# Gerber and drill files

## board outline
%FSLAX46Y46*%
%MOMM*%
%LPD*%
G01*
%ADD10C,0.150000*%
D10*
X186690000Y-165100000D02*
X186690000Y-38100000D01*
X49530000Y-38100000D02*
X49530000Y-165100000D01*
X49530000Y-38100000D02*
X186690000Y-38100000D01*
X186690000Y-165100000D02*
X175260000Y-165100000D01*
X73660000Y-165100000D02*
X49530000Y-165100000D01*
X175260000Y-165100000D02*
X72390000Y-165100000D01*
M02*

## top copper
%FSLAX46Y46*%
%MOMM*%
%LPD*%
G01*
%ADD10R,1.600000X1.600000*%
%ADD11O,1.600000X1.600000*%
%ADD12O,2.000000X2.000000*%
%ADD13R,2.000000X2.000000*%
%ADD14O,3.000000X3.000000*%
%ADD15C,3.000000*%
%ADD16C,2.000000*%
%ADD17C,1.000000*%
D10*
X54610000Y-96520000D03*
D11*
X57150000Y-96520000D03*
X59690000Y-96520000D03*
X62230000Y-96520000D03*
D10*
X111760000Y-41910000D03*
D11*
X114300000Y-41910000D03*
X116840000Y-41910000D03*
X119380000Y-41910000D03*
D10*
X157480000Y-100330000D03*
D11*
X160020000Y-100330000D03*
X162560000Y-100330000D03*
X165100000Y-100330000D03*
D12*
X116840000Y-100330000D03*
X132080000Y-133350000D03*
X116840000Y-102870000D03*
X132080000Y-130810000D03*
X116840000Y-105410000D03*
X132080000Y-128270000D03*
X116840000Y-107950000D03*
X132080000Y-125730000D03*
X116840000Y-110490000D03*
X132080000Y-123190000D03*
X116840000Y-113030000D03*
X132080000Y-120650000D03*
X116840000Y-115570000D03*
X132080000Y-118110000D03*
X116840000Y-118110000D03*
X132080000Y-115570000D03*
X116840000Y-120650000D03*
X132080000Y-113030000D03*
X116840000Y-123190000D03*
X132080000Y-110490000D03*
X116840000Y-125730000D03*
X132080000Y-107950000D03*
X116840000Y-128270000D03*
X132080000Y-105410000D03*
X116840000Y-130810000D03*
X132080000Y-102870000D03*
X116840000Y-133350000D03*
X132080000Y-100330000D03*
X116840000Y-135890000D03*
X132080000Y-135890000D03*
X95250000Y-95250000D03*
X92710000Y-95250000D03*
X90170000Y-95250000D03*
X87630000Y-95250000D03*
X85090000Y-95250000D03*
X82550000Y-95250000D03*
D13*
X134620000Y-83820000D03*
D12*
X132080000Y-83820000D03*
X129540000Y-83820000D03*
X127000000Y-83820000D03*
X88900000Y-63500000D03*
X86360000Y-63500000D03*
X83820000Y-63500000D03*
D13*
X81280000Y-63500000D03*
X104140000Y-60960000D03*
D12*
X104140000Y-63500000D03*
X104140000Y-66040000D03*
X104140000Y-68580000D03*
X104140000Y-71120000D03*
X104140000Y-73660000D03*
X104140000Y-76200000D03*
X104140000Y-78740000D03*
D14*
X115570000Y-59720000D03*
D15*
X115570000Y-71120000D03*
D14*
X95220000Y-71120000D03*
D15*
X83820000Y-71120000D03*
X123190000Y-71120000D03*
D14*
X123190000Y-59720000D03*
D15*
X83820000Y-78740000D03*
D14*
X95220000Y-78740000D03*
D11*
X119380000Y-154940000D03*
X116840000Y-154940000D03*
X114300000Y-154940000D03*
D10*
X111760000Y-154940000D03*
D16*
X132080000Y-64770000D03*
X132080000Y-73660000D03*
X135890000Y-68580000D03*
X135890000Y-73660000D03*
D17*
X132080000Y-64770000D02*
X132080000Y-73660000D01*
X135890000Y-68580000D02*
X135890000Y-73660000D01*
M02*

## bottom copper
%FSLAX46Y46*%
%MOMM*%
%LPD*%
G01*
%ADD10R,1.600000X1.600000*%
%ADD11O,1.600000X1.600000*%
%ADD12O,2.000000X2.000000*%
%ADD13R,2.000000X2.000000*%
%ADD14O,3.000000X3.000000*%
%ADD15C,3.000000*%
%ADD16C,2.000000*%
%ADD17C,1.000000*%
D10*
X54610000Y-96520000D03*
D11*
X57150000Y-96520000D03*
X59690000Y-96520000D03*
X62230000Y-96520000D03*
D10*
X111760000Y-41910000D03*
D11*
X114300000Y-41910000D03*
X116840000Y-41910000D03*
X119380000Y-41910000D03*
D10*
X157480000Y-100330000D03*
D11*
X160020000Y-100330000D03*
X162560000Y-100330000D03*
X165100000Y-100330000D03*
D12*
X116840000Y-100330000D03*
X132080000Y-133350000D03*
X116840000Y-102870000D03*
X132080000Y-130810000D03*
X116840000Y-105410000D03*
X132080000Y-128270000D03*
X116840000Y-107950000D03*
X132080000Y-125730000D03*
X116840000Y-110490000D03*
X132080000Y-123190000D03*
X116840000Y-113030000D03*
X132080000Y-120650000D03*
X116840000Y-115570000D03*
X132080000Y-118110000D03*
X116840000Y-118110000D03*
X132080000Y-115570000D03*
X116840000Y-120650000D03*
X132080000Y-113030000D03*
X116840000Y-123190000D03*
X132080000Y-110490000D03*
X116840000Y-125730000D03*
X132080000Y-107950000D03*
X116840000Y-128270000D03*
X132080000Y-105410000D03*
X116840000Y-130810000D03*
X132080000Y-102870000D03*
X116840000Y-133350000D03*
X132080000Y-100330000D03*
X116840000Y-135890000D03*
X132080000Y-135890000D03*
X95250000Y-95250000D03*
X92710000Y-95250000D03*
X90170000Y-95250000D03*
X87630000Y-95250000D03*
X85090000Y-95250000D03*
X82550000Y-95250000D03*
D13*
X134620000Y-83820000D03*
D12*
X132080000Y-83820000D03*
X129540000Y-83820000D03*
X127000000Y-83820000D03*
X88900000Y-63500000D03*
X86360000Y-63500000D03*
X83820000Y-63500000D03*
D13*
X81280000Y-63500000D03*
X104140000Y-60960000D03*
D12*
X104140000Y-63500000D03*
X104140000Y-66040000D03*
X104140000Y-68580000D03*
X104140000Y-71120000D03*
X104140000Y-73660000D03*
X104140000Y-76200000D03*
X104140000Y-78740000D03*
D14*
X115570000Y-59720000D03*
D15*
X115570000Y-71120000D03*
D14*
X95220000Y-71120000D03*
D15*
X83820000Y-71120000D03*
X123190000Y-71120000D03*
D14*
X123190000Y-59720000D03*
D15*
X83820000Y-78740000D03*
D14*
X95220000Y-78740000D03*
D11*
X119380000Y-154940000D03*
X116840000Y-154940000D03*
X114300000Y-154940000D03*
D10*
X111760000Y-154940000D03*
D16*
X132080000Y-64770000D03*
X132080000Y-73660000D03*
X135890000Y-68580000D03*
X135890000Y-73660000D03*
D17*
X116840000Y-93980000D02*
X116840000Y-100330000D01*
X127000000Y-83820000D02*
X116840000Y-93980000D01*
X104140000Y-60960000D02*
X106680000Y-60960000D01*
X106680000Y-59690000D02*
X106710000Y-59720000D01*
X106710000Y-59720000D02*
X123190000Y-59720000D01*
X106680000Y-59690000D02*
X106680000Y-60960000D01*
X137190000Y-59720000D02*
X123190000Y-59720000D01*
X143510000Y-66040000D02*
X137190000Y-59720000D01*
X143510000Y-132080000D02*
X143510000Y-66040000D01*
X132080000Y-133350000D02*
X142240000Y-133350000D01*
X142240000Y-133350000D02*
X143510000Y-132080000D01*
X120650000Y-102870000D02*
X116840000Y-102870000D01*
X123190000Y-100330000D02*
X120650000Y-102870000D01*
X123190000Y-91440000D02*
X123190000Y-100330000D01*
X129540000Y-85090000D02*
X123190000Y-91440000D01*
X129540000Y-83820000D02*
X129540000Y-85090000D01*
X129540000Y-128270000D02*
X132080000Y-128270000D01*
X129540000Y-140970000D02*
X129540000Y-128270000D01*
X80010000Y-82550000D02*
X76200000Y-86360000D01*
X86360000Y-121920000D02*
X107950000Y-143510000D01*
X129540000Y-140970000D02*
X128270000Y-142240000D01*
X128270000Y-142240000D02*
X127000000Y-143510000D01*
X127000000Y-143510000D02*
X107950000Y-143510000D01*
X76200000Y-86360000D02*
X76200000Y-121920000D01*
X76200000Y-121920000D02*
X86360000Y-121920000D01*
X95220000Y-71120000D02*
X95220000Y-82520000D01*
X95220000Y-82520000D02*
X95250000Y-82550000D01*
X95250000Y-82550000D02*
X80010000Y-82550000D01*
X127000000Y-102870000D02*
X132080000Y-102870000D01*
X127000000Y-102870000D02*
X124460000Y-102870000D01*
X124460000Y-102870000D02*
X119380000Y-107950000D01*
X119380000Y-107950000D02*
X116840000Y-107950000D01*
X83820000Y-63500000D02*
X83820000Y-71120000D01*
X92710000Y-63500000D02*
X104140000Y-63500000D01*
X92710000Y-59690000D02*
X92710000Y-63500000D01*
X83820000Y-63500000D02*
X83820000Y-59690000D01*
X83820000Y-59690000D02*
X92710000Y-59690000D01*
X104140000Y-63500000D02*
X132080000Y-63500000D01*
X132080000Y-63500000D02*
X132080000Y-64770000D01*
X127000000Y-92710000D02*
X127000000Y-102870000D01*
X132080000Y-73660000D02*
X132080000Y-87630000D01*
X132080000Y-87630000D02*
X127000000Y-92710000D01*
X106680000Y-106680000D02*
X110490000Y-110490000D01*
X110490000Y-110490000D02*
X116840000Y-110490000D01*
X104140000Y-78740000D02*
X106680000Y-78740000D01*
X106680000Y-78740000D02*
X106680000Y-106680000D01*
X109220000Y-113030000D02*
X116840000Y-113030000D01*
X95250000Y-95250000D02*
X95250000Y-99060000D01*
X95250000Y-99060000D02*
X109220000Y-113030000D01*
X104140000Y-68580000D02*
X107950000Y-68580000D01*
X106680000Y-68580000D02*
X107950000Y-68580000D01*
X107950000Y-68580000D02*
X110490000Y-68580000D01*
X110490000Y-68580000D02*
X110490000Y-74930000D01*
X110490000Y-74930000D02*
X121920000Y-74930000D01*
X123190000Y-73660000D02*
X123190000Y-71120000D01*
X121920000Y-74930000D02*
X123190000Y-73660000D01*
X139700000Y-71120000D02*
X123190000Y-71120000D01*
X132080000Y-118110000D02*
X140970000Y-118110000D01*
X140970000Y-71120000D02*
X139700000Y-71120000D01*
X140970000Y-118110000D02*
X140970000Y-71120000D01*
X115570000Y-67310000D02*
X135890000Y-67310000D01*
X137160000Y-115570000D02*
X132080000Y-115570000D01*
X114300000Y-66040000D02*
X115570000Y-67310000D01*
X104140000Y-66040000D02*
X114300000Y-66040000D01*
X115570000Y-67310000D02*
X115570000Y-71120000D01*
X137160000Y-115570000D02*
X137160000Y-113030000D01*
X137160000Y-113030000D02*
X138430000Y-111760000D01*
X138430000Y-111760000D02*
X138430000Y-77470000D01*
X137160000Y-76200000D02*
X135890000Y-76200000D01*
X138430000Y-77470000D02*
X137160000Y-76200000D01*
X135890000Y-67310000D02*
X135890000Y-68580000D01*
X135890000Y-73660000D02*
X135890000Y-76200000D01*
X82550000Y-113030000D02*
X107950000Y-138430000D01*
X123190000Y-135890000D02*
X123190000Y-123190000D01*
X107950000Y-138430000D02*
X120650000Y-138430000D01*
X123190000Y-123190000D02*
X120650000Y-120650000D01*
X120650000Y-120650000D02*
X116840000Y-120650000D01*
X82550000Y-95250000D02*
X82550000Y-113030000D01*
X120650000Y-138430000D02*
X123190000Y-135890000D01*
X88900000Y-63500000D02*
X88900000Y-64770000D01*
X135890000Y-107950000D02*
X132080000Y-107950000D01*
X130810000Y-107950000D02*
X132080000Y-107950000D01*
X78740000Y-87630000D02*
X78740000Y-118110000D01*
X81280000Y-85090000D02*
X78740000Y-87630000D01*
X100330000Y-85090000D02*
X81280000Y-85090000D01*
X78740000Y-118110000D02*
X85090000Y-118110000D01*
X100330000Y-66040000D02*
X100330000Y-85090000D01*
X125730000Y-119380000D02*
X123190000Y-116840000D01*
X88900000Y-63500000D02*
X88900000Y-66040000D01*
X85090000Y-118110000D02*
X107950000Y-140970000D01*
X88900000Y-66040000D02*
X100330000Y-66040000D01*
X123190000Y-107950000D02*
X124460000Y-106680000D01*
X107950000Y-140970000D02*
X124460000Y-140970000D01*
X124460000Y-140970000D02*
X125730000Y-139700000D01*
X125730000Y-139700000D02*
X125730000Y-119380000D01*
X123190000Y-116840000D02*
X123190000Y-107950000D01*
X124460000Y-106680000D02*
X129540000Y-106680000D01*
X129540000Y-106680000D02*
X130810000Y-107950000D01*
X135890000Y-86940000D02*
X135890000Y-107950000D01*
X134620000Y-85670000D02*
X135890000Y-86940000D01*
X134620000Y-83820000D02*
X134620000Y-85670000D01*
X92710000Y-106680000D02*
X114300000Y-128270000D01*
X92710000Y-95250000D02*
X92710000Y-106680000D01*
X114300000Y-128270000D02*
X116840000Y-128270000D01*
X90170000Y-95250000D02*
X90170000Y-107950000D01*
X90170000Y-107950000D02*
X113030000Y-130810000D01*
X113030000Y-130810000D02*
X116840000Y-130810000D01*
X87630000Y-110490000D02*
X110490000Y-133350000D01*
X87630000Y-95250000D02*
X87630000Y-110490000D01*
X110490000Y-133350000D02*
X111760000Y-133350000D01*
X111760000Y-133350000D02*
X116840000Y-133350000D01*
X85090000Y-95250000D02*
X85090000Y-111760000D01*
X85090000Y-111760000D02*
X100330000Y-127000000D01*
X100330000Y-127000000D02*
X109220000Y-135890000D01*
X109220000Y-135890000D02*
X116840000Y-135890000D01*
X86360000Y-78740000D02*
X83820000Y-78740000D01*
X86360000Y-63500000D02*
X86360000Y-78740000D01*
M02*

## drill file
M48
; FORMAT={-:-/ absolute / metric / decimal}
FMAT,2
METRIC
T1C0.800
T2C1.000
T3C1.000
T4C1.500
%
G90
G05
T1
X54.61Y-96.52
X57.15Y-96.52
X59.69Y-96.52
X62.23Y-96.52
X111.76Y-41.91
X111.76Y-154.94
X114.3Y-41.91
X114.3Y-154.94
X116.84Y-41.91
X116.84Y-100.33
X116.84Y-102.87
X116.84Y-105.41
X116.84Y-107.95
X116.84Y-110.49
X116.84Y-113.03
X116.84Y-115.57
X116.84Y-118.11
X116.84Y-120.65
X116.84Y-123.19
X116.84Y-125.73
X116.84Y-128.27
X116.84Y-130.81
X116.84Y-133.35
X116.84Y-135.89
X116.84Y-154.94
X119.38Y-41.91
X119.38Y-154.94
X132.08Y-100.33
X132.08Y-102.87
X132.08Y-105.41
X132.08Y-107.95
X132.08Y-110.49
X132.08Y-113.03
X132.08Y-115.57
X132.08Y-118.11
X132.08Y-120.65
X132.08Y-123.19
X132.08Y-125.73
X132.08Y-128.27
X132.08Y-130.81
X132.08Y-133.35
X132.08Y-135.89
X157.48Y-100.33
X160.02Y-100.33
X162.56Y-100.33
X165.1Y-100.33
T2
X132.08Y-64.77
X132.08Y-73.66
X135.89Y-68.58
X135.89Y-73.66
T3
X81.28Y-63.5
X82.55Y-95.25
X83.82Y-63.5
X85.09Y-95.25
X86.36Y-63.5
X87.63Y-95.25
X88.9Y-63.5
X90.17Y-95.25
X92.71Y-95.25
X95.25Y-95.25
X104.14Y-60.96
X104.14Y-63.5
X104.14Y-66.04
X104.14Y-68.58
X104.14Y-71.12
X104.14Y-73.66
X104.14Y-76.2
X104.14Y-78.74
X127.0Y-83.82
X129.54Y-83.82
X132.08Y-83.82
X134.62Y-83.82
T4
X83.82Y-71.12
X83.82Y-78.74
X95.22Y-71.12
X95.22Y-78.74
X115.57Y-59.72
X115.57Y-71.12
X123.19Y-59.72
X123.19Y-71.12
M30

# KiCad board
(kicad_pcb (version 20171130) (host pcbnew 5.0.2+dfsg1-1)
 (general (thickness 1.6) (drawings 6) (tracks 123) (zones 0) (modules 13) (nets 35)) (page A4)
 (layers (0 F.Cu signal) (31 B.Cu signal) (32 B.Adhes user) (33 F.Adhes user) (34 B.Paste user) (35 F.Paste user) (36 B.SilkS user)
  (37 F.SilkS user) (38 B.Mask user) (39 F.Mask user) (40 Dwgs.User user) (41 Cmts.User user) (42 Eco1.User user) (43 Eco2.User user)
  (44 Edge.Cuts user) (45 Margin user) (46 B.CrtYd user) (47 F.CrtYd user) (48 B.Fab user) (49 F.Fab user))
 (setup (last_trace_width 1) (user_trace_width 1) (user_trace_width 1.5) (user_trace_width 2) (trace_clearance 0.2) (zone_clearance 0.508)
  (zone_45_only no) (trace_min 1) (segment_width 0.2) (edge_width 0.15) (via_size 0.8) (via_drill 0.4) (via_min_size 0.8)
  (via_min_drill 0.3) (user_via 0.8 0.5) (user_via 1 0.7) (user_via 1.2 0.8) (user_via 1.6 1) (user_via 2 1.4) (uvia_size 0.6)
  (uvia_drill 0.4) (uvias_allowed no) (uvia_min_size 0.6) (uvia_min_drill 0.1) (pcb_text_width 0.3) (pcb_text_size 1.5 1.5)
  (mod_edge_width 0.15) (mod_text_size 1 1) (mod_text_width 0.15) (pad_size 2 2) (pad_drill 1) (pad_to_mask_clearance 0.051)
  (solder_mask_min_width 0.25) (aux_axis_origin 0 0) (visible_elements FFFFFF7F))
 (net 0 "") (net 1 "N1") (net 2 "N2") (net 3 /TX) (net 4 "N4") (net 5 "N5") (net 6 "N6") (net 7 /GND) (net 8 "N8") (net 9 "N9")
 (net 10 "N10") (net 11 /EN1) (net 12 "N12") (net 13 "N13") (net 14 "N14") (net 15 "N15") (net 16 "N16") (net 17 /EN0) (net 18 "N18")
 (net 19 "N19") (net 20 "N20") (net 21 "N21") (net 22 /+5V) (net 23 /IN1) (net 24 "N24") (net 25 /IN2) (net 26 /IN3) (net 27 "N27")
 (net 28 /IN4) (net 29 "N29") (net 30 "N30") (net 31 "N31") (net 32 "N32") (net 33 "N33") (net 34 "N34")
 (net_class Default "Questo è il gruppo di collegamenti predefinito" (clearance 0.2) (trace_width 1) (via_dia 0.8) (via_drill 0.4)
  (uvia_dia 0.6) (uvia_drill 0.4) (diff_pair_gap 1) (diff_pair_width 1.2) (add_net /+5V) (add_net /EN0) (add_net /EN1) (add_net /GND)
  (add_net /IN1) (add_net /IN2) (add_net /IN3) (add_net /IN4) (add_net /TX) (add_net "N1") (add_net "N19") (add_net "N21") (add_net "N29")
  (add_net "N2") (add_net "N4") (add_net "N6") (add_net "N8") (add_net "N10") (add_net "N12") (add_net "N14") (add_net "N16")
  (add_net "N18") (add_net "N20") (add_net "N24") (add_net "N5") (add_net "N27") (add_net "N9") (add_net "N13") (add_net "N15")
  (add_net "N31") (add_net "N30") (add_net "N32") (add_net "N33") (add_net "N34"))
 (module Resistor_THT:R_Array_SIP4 (layer F.Cu) (at 54.61 96.52)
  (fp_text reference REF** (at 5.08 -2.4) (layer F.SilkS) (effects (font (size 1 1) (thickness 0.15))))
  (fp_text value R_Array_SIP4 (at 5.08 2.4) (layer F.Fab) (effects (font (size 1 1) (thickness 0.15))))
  (pad 1 thru_hole rect (at 0 0) (size 1.6 1.6) (drill 0.8) (layers *.Cu *.Mask))
  (pad 2 thru_hole oval (at 2.54 0) (size 1.6 1.6) (drill 0.8) (layers *.Cu *.Mask))
  (pad 3 thru_hole oval (at 5.08 0) (size 1.6 1.6) (drill 0.8) (layers *.Cu *.Mask))
  (pad 4 thru_hole oval (at 7.62 0) (size 1.6 1.6) (drill 0.8) (layers *.Cu *.Mask)))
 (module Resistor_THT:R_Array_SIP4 (layer F.Cu) (at 111.76 41.91)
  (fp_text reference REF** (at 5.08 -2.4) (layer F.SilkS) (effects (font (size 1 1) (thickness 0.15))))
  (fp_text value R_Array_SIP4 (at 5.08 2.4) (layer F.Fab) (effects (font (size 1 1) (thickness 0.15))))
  (pad 1 thru_hole rect (at 0 0) (size 1.6 1.6) (drill 0.8) (layers *.Cu *.Mask))
  (pad 2 thru_hole oval (at 2.54 0) (size 1.6 1.6) (drill 0.8) (layers *.Cu *.Mask))
  (pad 3 thru_hole oval (at 5.08 0) (size 1.6 1.6) (drill 0.8) (layers *.Cu *.Mask))
  (pad 4 thru_hole oval (at 7.62 0) (size 1.6 1.6) (drill 0.8) (layers *.Cu *.Mask)))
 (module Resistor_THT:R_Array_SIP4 (layer F.Cu) (at 157.48 100.33)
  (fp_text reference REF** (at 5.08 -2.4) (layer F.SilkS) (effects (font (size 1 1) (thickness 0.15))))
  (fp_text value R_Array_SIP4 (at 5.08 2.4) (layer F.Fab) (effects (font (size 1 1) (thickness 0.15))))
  (pad 1 thru_hole rect (at 0 0) (size 1.6 1.6) (drill 0.8) (layers *.Cu *.Mask))
  (pad 2 thru_hole oval (at 2.54 0) (size 1.6 1.6) (drill 0.8) (layers *.Cu *.Mask))
  (pad 3 thru_hole oval (at 5.08 0) (size 1.6 1.6) (drill 0.8) (layers *.Cu *.Mask))
  (pad 4 thru_hole oval (at 7.62 0) (size 1.6 1.6) (drill 0.8) (layers *.Cu *.Mask)))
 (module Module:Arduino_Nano (layer F.Cu) (at 116.84 100.33)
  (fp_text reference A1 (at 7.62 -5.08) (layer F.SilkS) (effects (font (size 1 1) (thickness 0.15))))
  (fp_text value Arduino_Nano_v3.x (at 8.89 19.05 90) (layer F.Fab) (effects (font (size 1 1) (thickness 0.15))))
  (pad 1 thru_hole oval (at 0 0) (size 2 2) (drill 0.8) (layers *.Cu *.Mask) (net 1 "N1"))
  (pad 17 thru_hole oval (at 15.24 33.02) (size 2 2) (drill 0.8) (layers *.Cu *.Mask) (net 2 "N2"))
  (pad 2 thru_hole oval (at 0 2.54) (size 2 2) (drill 0.8) (layers *.Cu *.Mask) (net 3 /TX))
  (pad 18 thru_hole oval (at 15.24 30.48) (size 2 2) (drill 0.8) (layers *.Cu *.Mask) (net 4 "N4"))
  (pad 3 thru_hole oval (at 0 5.08) (size 2 2) (drill 0.8) (layers *.Cu *.Mask) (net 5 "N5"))
  (pad 19 thru_hole oval (at 15.24 27.94) (size 2 2) (drill 0.8) (layers *.Cu *.Mask) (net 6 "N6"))
  (pad 4 thru_hole oval (at 0 7.62) (size 2 2) (drill 0.8) (layers *.Cu *.Mask) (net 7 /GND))
  (pad 20 thru_hole oval (at 15.24 25.4) (size 2 2) (drill 0.8) (layers *.Cu *.Mask) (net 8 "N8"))
  (pad 5 thru_hole oval (at 0 10.16) (size 2 2) (drill 0.8) (layers *.Cu *.Mask) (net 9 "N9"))
  (pad 21 thru_hole oval (at 15.24 22.86) (size 2 2) (drill 0.8) (layers *.Cu *.Mask) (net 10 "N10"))
  (pad 6 thru_hole oval (at 0 12.7) (size 2 2) (drill 0.8) (layers *.Cu *.Mask) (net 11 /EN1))
  (pad 22 thru_hole oval (at 15.24 20.32) (size 2 2) (drill 0.8) (layers *.Cu *.Mask) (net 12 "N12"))
  (pad 7 thru_hole oval (at 0 15.24) (size 2 2) (drill 0.8) (layers *.Cu *.Mask) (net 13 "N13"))
  (pad 23 thru_hole oval (at 15.24 17.78) (size 2 2) (drill 0.8) (layers *.Cu *.Mask) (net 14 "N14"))
  (pad 8 thru_hole oval (at 0 17.78) (size 2 2) (drill 0.8) (layers *.Cu *.Mask) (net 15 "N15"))
  (pad 24 thru_hole oval (at 15.24 15.24) (size 2 2) (drill 0.8) (layers *.Cu *.Mask) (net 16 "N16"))
  (pad 9 thru_hole oval (at 0 20.32) (size 2 2) (drill 0.8) (layers *.Cu *.Mask) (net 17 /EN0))
  (pad 25 thru_hole oval (at 15.24 12.7) (size 2 2) (drill 0.8) (layers *.Cu *.Mask) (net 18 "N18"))
  (pad 10 thru_hole oval (at 0 22.86) (size 2 2) (drill 0.8) (layers *.Cu *.Mask) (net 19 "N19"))
  (pad 26 thru_hole oval (at 15.24 10.16) (size 2 2) (drill 0.8) (layers *.Cu *.Mask) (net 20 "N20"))
  (pad 11 thru_hole oval (at 0 25.4) (size 2 2) (drill 0.8) (layers *.Cu *.Mask) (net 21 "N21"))
  (pad 27 thru_hole oval (at 15.24 7.62) (size 2 2) (drill 0.8) (layers *.Cu *.Mask) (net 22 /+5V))
  (pad 12 thru_hole oval (at 0 27.94) (size 2 2) (drill 0.8) (layers *.Cu *.Mask) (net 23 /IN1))
  (pad 28 thru_hole oval (at 15.24 5.08) (size 2 2) (drill 0.8) (layers *.Cu *.Mask) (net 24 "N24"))
  (pad 13 thru_hole oval (at 0 30.48) (size 2 2) (drill 0.8) (layers *.Cu *.Mask) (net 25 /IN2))
  (pad 29 thru_hole oval (at 15.24 2.54) (size 2 2) (drill 0.8) (layers *.Cu *.Mask) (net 7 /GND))
  (pad 14 thru_hole oval (at 0 33.02) (size 2 2) (drill 0.8) (layers *.Cu *.Mask) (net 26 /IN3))
  (pad 30 thru_hole oval (at 15.24 0) (size 2 2) (drill 0.8) (layers *.Cu *.Mask) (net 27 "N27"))
  (pad 15 thru_hole oval (at 0 35.56) (size 2 2) (drill 0.8) (layers *.Cu *.Mask) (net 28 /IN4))
  (pad 16 thru_hole oval (at 15.24 35.56) (size 2 2) (drill 0.8) (layers *.Cu *.Mask) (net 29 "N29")))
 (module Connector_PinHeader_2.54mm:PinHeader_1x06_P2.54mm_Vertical (layer F.Cu) (at 95.25 95.25 270)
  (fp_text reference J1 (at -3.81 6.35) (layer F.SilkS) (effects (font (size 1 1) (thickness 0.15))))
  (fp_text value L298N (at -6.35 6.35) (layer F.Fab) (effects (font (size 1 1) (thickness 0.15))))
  (pad 1 thru_hole oval (at 0 0 270) (size 2 2) (drill 1) (layers *.Cu *.Mask) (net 11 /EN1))
  (pad 2 thru_hole oval (at 0 2.54 270) (size 2 2) (drill 1) (layers *.Cu *.Mask) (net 23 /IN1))
  (pad 3 thru_hole oval (at 0 5.08 270) (size 2 2) (drill 1) (layers *.Cu *.Mask) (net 25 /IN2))
  (pad 4 thru_hole oval (at 0 7.62 270) (size 2 2) (drill 1) (layers *.Cu *.Mask) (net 26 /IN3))
  (pad 5 thru_hole oval (at 0 10.16 270) (size 2 2) (drill 1) (layers *.Cu *.Mask) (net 28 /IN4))
  (pad 6 thru_hole oval (at 0 12.7 270) (size 2 2) (drill 1) (layers *.Cu *.Mask) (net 17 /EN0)))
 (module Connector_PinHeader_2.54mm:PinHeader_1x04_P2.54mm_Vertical (layer F.Cu) (at 134.62 83.82 270)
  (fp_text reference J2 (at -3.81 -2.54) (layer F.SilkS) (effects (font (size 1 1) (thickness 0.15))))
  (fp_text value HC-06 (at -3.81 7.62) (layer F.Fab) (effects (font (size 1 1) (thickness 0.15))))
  (pad 1 thru_hole rect (at 0 0 270) (size 2 2) (drill 1) (layers *.Cu *.Mask) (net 22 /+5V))
  (pad 2 thru_hole oval (at 0 2.54 270) (size 2 2) (drill 1) (layers *.Cu *.Mask) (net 7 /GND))
  (pad 3 thru_hole oval (at 0 5.08 270) (size 2 2) (drill 1) (layers *.Cu *.Mask) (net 3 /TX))
  (pad 4 thru_hole oval (at 0 7.62 270) (size 2 2) (drill 1) (layers *.Cu *.Mask) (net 1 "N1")))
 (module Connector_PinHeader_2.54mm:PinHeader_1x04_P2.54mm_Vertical (layer F.Cu) (at 81.28 63.5 90)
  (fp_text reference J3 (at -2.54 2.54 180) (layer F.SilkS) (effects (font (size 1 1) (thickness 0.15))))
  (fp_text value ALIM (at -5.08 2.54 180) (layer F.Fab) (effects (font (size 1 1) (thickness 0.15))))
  (pad 4 thru_hole oval (at 0 7.62 90) (size 2 2) (drill 1) (layers *.Cu *.Mask) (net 22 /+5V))
  (pad 3 thru_hole oval (at 0 5.08 90) (size 2 2) (drill 1) (layers *.Cu *.Mask) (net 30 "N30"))
  (pad 2 thru_hole oval (at 0 2.54 90) (size 2 2) (drill 1) (layers *.Cu *.Mask) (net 7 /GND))
  (pad 1 thru_hole rect (at 0 0 90) (size 2 2) (drill 1) (layers *.Cu *.Mask) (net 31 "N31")))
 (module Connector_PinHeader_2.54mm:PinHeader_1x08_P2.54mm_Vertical (layer F.Cu) (at 104.14 60.96)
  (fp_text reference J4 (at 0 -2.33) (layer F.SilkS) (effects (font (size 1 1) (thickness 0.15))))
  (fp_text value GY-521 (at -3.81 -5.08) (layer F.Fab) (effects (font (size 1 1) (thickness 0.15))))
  (pad 1 thru_hole rect (at 0 0) (size 2 2) (drill 1) (layers *.Cu *.Mask) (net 2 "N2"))
  (pad 2 thru_hole oval (at 0 2.54) (size 2 2) (drill 1) (layers *.Cu *.Mask) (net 7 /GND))
  (pad 3 thru_hole oval (at 0 5.08) (size 2 2) (drill 1) (layers *.Cu *.Mask) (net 16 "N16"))
  (pad 4 thru_hole oval (at 0 7.62) (size 2 2) (drill 1) (layers *.Cu *.Mask) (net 14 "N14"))
  (pad 5 thru_hole oval (at 0 10.16) (size 2 2) (drill 1) (layers *.Cu *.Mask) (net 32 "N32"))
  (pad 6 thru_hole oval (at 0 12.7) (size 2 2) (drill 1) (layers *.Cu *.Mask) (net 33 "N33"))
  (pad 7 thru_hole oval (at 0 15.24) (size 2 2) (drill 1) (layers *.Cu *.Mask) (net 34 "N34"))
  (pad 8 thru_hole oval (at 0 17.78) (size 2 2) (drill 1) (layers *.Cu *.Mask) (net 9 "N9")))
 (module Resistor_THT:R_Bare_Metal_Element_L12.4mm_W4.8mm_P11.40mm (layer F.Cu) (at 115.57 71.12 90)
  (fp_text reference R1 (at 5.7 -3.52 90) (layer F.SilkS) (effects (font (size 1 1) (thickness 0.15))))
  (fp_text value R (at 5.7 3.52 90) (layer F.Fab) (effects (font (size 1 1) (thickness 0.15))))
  (pad 2 thru_hole oval (at 11.4 0 90) (size 3 3) (drill 1.5) (layers *.Cu *.Mask) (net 2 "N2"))
  (pad 1 thru_hole circle (at 0 0 90) (size 3 3) (drill 1.5) (layers *.Cu *.Mask) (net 16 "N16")))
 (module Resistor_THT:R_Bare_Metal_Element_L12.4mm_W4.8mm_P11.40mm (layer F.Cu) (at 83.82 71.12)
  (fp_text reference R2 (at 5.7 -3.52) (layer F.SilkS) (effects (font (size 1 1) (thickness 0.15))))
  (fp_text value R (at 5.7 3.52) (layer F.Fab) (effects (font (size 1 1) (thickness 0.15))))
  (pad 2 thru_hole oval (at 11.4 0) (size 3 3) (drill 1.5) (layers *.Cu *.Mask) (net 6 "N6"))
  (pad 1 thru_hole circle (at 0 0) (size 3 3) (drill 1.5) (layers *.Cu *.Mask) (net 7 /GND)))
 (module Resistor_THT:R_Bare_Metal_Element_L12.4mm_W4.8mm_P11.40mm (layer F.Cu) (at 123.19 71.12 90)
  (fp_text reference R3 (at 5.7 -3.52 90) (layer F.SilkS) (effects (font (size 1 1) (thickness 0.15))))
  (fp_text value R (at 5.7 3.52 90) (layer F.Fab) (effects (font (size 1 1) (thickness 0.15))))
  (pad 1 thru_hole circle (at 0 0 90) (size 3 3) (drill 1.5) (layers *.Cu *.Mask) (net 14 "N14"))
  (pad 2 thru_hole oval (at 11.4 0 90) (size 3 3) (drill 1.5) (layers *.Cu *.Mask) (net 2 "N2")))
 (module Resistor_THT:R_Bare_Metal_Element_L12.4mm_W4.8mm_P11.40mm (layer F.Cu) (at 83.82 78.74)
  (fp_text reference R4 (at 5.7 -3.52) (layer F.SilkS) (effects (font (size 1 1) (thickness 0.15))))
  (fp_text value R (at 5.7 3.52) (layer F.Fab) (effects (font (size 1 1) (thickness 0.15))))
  (pad 1 thru_hole circle (at 0 0) (size 3 3) (drill 1.5) (layers *.Cu *.Mask) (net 30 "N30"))
  (pad 2 thru_hole oval (at 11.4 0) (size 3 3) (drill 1.5) (layers *.Cu *.Mask) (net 6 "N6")))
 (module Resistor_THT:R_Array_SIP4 (layer F.Cu) (at 111.76 154.94)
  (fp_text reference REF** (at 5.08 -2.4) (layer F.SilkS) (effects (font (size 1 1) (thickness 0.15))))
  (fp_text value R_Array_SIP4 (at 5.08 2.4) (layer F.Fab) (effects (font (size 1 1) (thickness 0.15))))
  (pad 4 thru_hole oval (at 7.62 0) (size 1.6 1.6) (drill 0.8) (layers *.Cu *.Mask))
  (pad 3 thru_hole oval (at 5.08 0) (size 1.6 1.6) (drill 0.8) (layers *.Cu *.Mask))
  (pad 2 thru_hole oval (at 2.54 0) (size 1.6 1.6) (drill 0.8) (layers *.Cu *.Mask))
  (pad 1 thru_hole rect (at 0 0) (size 1.6 1.6) (drill 0.8) (layers *.Cu *.Mask)))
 (gr_line (start 186.69 165.1) (end 186.69 38.1) (layer Edge.Cuts) (width 0.15))
 (gr_line (start 49.53 38.1) (end 49.53 165.1) (layer Edge.Cuts) (width 0.15))
 (gr_line (start 49.53 38.1) (end 186.69 38.1) (layer Edge.Cuts) (width 0.15))
 (gr_line (start 186.69 165.1) (end 175.26 165.1) (layer Edge.Cuts) (width 0.15))
 (gr_line (start 73.66 165.1) (end 49.53 165.1) (layer Edge.Cuts) (width 0.15))
 (gr_line (start 175.26 165.1) (end 72.39 165.1) (layer Edge.Cuts) (width 0.15))
 (segment (start 116.84 93.98) (end 116.84 100.33) (width 1) (layer B.Cu) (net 1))
 (segment (start 127 83.82) (end 116.84 93.98) (width 1) (layer B.Cu) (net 1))
 (segment (start 104.14 60.96) (end 106.68 60.96) (width 1) (layer B.Cu) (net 2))
 (segment (start 106.68 59.69) (end 106.71 59.72) (width 1) (layer B.Cu) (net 2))
 (segment (start 106.71 59.72) (end 123.19 59.72) (width 1) (layer B.Cu) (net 2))
 (segment (start 106.68 59.69) (end 106.68 60.96) (width 1) (layer B.Cu) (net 2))
 (segment (start 137.19 59.72) (end 123.19 59.72) (width 1) (layer B.Cu) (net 2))
 (segment (start 143.51 66.04) (end 137.19 59.72) (width 1) (layer B.Cu) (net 2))
 (segment (start 143.51 132.08) (end 143.51 66.04) (width 1) (layer B.Cu) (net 2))
 (segment (start 132.08 133.35) (end 142.24 133.35) (width 1) (layer B.Cu) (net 2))
 (segment (start 142.24 133.35) (end 143.51 132.08) (width 1) (layer B.Cu) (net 2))
 (segment (start 120.65 102.87) (end 116.84 102.87) (width 1) (layer B.Cu) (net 3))
 (segment (start 123.19 100.33) (end 120.65 102.87) (width 1) (layer B.Cu) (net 3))
 (segment (start 123.19 91.44) (end 123.19 100.33) (width 1) (layer B.Cu) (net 3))
 (segment (start 129.54 85.09) (end 123.19 91.44) (width 1) (layer B.Cu) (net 3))
 (segment (start 129.54 83.82) (end 129.54 85.09) (width 1) (layer B.Cu) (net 3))
 (segment (start 129.54 128.27) (end 132.08 128.27) (width 1) (layer B.Cu) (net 6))
 (segment (start 129.54 140.97) (end 129.54 128.27) (width 1) (layer B.Cu) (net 6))
 (segment (start 80.01 82.55) (end 76.2 86.36) (width 1) (layer B.Cu) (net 6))
 (segment (start 86.36 121.92) (end 107.95 143.51) (width 1) (layer B.Cu) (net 6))
 (segment (start 129.54 140.97) (end 128.27 142.24) (width 1) (layer B.Cu) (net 6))
 (segment (start 128.27 142.24) (end 127 143.51) (width 1) (layer B.Cu) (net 6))
 (segment (start 127 143.51) (end 107.95 143.51) (width 1) (layer B.Cu) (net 6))
 (segment (start 76.2 86.36) (end 76.2 121.92) (width 1) (layer B.Cu) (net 6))
 (segment (start 76.2 121.92) (end 86.36 121.92) (width 1) (layer B.Cu) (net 6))
 (segment (start 95.22 71.12) (end 95.22 82.52) (width 1) (layer B.Cu) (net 6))
 (segment (start 95.22 82.52) (end 95.25 82.55) (width 1) (layer B.Cu) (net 6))
 (segment (start 95.25 82.55) (end 80.01 82.55) (width 1) (layer B.Cu) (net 6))
 (segment (start 127 102.87) (end 132.08 102.87) (width 1) (layer B.Cu) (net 7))
 (segment (start 127 102.87) (end 124.46 102.87) (width 1) (layer B.Cu) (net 7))
 (segment (start 124.46 102.87) (end 119.38 107.95) (width 1) (layer B.Cu) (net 7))
 (segment (start 119.38 107.95) (end 116.84 107.95) (width 1) (layer B.Cu) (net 7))
 (segment (start 83.82 63.5) (end 83.82 71.12) (width 1) (layer B.Cu) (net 7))
 (segment (start 92.71 63.5) (end 104.14 63.5) (width 1) (layer B.Cu) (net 7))
 (segment (start 92.71 59.69) (end 92.71 63.5) (width 1) (layer B.Cu) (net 7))
 (segment (start 83.82 63.5) (end 83.82 59.69) (width 1) (layer B.Cu) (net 7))
 (segment (start 83.82 59.69) (end 92.71 59.69) (width 1) (layer B.Cu) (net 7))
 (segment (start 104.14 63.5) (end 132.08 63.5) (width 1) (layer B.Cu) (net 7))
 (via (at 132.08 64.77) (size 2) (drill 1) (layers F.Cu B.Cu) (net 7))
 (segment (start 132.08 63.5) (end 132.08 64.77) (width 1) (layer B.Cu) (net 7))
 (via (at 132.08 73.66) (size 2) (drill 1) (layers F.Cu B.Cu) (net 7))
 (segment (start 132.08 64.77) (end 132.08 73.66) (width 1) (layer F.Cu) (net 7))
 (segment (start 127 92.71) (end 127 102.87) (width 1) (layer B.Cu) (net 7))
 (segment (start 132.08 73.66) (end 132.08 87.63) (width 1) (layer B.Cu) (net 7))
 (segment (start 132.08 87.63) (end 127 92.71) (width 1) (layer B.Cu) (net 7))
 (segment (start 106.68 106.68) (end 110.49 110.49) (width 1) (layer B.Cu) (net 9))
 (segment (start 110.49 110.49) (end 116.84 110.49) (width 1) (layer B.Cu) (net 9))
 (segment (start 104.14 78.74) (end 106.68 78.74) (width 1) (layer B.Cu) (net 9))
 (segment (start 106.68 78.74) (end 106.68 106.68) (width 1) (layer B.Cu) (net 9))
 (segment (start 109.22 113.03) (end 116.84 113.03) (width 1) (layer B.Cu) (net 11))
 (segment (start 95.25 95.25) (end 95.25 99.06) (width 1) (layer B.Cu) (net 11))
 (segment (start 95.25 99.06) (end 109.22 113.03) (width 1) (layer B.Cu) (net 11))
 (segment (start 104.14 68.58) (end 107.95 68.58) (width 1) (layer B.Cu) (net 14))
 (segment (start 106.68 68.58) (end 107.95 68.58) (width 1) (layer B.Cu) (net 14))
 (segment (start 107.95 68.58) (end 110.49 68.58) (width 1) (layer B.Cu) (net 14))
 (segment (start 110.49 68.58) (end 110.49 74.93) (width 1) (layer B.Cu) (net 14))
 (segment (start 110.49 74.93) (end 121.92 74.93) (width 1) (layer B.Cu) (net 14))
 (segment (start 123.19 73.66) (end 123.19 71.12) (width 1) (layer B.Cu) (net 14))
 (segment (start 121.92 74.93) (end 123.19 73.66) (width 1) (layer B.Cu) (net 14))
 (segment (start 139.7 71.12) (end 123.19 71.12) (width 1) (layer B.Cu) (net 14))
 (segment (start 132.08 118.11) (end 140.97 118.11) (width 1) (layer B.Cu) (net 14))
 (segment (start 140.97 71.12) (end 139.7 71.12) (width 1) (layer B.Cu) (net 14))
 (segment (start 140.97 118.11) (end 140.97 71.12) (width 1) (layer B.Cu) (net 14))
 (segment (start 115.57 67.31) (end 135.89 67.31) (width 1) (layer B.Cu) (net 16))
 (segment (start 137.16 115.57) (end 132.08 115.57) (width 1) (layer B.Cu) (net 16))
 (segment (start 114.3 66.04) (end 115.57 67.31) (width 1) (layer B.Cu) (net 16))
 (segment (start 104.14 66.04) (end 114.3 66.04) (width 1) (layer B.Cu) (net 16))
 (segment (start 115.57 67.31) (end 115.57 71.12) (width 1) (layer B.Cu) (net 16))
 (segment (start 137.16 115.57) (end 137.16 113.03) (width 1) (layer B.Cu) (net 16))
 (segment (start 137.16 113.03) (end 138.43 111.76) (width 1) (layer B.Cu) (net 16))
 (segment (start 138.43 111.76) (end 138.43 77.47) (width 1) (layer B.Cu) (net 16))
 (segment (start 137.16 76.2) (end 135.89 76.2) (width 1) (layer B.Cu) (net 16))
 (segment (start 138.43 77.47) (end 137.16 76.2) (width 1) (layer B.Cu) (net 16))
 (via (at 135.89 68.58) (size 2) (drill 1) (layers F.Cu B.Cu) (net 16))
 (segment (start 135.89 67.31) (end 135.89 68.58) (width 1) (layer B.Cu) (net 16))
 (via (at 135.89 73.66) (size 2) (drill 1) (layers F.Cu B.Cu) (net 16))
 (segment (start 135.89 68.58) (end 135.89 73.66) (width 1) (layer F.Cu) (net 16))
 (segment (start 135.89 73.66) (end 135.89 76.2) (width 1) (layer B.Cu) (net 16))
 (segment (start 82.55 113.03) (end 107.95 138.43) (width 1) (layer B.Cu) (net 17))
 (segment (start 123.19 135.89) (end 123.19 123.19) (width 1) (layer B.Cu) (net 17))
 (segment (start 107.95 138.43) (end 120.65 138.43) (width 1) (layer B.Cu) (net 17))
 (segment (start 123.19 123.19) (end 120.65 120.65) (width 1) (layer B.Cu) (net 17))
 (segment (start 120.65 120.65) (end 116.84 120.65) (width 1) (layer B.Cu) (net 17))
 (segment (start 82.55 95.25) (end 82.55 113.03) (width 1) (layer B.Cu) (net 17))
 (segment (start 120.65 138.43) (end 123.19 135.89) (width 1) (layer B.Cu) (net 17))
 (segment (start 88.9 63.5) (end 88.9 64.77) (width 1) (layer B.Cu) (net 22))
 (segment (start 135.89 107.95) (end 132.08 107.95) (width 1) (layer B.Cu) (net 22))
 (segment (start 130.81 107.95) (end 132.08 107.95) (width 1) (layer B.Cu) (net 22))
 (segment (start 78.74 87.63) (end 78.74 118.11) (width 1) (layer B.Cu) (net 22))
 (segment (start 81.28 85.09) (end 78.74 87.63) (width 1) (layer B.Cu) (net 22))
 (segment (start 100.33 85.09) (end 81.28 85.09) (width 1) (layer B.Cu) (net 22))
 (segment (start 78.74 118.11) (end 85.09 118.11) (width 1) (layer B.Cu) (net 22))
 (segment (start 100.33 66.04) (end 100.33 85.09) (width 1) (layer B.Cu) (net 22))
 (segment (start 125.73 119.38) (end 123.19 116.84) (width 1) (layer B.Cu) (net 22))
 (segment (start 88.9 63.5) (end 88.9 66.04) (width 1) (layer B.Cu) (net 22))
 (segment (start 85.09 118.11) (end 107.95 140.97) (width 1) (layer B.Cu) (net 22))
 (segment (start 88.9 66.04) (end 100.33 66.04) (width 1) (layer B.Cu) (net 22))
 (segment (start 123.19 107.95) (end 124.46 106.68) (width 1) (layer B.Cu) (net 22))
 (segment (start 107.95 140.97) (end 124.46 140.97) (width 1) (layer B.Cu) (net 22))
 (segment (start 124.46 140.97) (end 125.73 139.7) (width 1) (layer B.Cu) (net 22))
 (segment (start 125.73 139.7) (end 125.73 119.38) (width 1) (layer B.Cu) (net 22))
 (segment (start 123.19 116.84) (end 123.19 107.95) (width 1) (layer B.Cu) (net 22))
 (segment (start 124.46 106.68) (end 129.54 106.68) (width 1) (layer B.Cu) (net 22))
 (segment (start 129.54 106.68) (end 130.81 107.95) (width 1) (layer B.Cu) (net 22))
 (segment (start 135.89 86.94) (end 135.89 107.95) (width 1) (layer B.Cu) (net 22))
 (segment (start 134.62 85.67) (end 135.89 86.94) (width 1) (layer B.Cu) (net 22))
 (segment (start 134.62 83.82) (end 134.62 85.67) (width 1) (layer B.Cu) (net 22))
 (segment (start 92.71 106.68) (end 114.3 128.27) (width 1) (layer B.Cu) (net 23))
 (segment (start 92.71 95.25) (end 92.71 106.68) (width 1) (layer B.Cu) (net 23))
 (segment (start 114.3 128.27) (end 116.84 128.27) (width 1) (layer B.Cu) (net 23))
 (segment (start 90.17 95.25) (end 90.17 107.95) (width 1) (layer B.Cu) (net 25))
 (segment (start 90.17 107.95) (end 113.03 130.81) (width 1) (layer B.Cu) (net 25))
 (segment (start 113.03 130.81) (end 116.84 130.81) (width 1) (layer B.Cu) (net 25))
 (segment (start 87.63 110.49) (end 110.49 133.35) (width 1) (layer B.Cu) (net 26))
 (segment (start 87.63 95.25) (end 87.63 110.49) (width 1) (layer B.Cu) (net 26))
 (segment (start 110.49 133.35) (end 111.76 133.35) (width 1) (layer B.Cu) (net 26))
 (segment (start 111.76 133.35) (end 116.84 133.35) (width 1) (layer B.Cu) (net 26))
 (segment (start 85.09 95.25) (end 85.09 111.76) (width 1) (layer B.Cu) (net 28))
 (segment (start 85.09 111.76) (end 100.33 127) (width 1) (layer B.Cu) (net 28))
 (segment (start 100.33 127) (end 109.22 135.89) (width 1) (layer B.Cu) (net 28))
 (segment (start 109.22 135.89) (end 116.84 135.89) (width 1) (layer B.Cu) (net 28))
 (segment (start 86.36 78.74) (end 83.82 78.74) (width 1) (layer B.Cu) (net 30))
 (segment (start 86.36 63.5) (end 86.36 78.74) (width 1) (layer B.Cu) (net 30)))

